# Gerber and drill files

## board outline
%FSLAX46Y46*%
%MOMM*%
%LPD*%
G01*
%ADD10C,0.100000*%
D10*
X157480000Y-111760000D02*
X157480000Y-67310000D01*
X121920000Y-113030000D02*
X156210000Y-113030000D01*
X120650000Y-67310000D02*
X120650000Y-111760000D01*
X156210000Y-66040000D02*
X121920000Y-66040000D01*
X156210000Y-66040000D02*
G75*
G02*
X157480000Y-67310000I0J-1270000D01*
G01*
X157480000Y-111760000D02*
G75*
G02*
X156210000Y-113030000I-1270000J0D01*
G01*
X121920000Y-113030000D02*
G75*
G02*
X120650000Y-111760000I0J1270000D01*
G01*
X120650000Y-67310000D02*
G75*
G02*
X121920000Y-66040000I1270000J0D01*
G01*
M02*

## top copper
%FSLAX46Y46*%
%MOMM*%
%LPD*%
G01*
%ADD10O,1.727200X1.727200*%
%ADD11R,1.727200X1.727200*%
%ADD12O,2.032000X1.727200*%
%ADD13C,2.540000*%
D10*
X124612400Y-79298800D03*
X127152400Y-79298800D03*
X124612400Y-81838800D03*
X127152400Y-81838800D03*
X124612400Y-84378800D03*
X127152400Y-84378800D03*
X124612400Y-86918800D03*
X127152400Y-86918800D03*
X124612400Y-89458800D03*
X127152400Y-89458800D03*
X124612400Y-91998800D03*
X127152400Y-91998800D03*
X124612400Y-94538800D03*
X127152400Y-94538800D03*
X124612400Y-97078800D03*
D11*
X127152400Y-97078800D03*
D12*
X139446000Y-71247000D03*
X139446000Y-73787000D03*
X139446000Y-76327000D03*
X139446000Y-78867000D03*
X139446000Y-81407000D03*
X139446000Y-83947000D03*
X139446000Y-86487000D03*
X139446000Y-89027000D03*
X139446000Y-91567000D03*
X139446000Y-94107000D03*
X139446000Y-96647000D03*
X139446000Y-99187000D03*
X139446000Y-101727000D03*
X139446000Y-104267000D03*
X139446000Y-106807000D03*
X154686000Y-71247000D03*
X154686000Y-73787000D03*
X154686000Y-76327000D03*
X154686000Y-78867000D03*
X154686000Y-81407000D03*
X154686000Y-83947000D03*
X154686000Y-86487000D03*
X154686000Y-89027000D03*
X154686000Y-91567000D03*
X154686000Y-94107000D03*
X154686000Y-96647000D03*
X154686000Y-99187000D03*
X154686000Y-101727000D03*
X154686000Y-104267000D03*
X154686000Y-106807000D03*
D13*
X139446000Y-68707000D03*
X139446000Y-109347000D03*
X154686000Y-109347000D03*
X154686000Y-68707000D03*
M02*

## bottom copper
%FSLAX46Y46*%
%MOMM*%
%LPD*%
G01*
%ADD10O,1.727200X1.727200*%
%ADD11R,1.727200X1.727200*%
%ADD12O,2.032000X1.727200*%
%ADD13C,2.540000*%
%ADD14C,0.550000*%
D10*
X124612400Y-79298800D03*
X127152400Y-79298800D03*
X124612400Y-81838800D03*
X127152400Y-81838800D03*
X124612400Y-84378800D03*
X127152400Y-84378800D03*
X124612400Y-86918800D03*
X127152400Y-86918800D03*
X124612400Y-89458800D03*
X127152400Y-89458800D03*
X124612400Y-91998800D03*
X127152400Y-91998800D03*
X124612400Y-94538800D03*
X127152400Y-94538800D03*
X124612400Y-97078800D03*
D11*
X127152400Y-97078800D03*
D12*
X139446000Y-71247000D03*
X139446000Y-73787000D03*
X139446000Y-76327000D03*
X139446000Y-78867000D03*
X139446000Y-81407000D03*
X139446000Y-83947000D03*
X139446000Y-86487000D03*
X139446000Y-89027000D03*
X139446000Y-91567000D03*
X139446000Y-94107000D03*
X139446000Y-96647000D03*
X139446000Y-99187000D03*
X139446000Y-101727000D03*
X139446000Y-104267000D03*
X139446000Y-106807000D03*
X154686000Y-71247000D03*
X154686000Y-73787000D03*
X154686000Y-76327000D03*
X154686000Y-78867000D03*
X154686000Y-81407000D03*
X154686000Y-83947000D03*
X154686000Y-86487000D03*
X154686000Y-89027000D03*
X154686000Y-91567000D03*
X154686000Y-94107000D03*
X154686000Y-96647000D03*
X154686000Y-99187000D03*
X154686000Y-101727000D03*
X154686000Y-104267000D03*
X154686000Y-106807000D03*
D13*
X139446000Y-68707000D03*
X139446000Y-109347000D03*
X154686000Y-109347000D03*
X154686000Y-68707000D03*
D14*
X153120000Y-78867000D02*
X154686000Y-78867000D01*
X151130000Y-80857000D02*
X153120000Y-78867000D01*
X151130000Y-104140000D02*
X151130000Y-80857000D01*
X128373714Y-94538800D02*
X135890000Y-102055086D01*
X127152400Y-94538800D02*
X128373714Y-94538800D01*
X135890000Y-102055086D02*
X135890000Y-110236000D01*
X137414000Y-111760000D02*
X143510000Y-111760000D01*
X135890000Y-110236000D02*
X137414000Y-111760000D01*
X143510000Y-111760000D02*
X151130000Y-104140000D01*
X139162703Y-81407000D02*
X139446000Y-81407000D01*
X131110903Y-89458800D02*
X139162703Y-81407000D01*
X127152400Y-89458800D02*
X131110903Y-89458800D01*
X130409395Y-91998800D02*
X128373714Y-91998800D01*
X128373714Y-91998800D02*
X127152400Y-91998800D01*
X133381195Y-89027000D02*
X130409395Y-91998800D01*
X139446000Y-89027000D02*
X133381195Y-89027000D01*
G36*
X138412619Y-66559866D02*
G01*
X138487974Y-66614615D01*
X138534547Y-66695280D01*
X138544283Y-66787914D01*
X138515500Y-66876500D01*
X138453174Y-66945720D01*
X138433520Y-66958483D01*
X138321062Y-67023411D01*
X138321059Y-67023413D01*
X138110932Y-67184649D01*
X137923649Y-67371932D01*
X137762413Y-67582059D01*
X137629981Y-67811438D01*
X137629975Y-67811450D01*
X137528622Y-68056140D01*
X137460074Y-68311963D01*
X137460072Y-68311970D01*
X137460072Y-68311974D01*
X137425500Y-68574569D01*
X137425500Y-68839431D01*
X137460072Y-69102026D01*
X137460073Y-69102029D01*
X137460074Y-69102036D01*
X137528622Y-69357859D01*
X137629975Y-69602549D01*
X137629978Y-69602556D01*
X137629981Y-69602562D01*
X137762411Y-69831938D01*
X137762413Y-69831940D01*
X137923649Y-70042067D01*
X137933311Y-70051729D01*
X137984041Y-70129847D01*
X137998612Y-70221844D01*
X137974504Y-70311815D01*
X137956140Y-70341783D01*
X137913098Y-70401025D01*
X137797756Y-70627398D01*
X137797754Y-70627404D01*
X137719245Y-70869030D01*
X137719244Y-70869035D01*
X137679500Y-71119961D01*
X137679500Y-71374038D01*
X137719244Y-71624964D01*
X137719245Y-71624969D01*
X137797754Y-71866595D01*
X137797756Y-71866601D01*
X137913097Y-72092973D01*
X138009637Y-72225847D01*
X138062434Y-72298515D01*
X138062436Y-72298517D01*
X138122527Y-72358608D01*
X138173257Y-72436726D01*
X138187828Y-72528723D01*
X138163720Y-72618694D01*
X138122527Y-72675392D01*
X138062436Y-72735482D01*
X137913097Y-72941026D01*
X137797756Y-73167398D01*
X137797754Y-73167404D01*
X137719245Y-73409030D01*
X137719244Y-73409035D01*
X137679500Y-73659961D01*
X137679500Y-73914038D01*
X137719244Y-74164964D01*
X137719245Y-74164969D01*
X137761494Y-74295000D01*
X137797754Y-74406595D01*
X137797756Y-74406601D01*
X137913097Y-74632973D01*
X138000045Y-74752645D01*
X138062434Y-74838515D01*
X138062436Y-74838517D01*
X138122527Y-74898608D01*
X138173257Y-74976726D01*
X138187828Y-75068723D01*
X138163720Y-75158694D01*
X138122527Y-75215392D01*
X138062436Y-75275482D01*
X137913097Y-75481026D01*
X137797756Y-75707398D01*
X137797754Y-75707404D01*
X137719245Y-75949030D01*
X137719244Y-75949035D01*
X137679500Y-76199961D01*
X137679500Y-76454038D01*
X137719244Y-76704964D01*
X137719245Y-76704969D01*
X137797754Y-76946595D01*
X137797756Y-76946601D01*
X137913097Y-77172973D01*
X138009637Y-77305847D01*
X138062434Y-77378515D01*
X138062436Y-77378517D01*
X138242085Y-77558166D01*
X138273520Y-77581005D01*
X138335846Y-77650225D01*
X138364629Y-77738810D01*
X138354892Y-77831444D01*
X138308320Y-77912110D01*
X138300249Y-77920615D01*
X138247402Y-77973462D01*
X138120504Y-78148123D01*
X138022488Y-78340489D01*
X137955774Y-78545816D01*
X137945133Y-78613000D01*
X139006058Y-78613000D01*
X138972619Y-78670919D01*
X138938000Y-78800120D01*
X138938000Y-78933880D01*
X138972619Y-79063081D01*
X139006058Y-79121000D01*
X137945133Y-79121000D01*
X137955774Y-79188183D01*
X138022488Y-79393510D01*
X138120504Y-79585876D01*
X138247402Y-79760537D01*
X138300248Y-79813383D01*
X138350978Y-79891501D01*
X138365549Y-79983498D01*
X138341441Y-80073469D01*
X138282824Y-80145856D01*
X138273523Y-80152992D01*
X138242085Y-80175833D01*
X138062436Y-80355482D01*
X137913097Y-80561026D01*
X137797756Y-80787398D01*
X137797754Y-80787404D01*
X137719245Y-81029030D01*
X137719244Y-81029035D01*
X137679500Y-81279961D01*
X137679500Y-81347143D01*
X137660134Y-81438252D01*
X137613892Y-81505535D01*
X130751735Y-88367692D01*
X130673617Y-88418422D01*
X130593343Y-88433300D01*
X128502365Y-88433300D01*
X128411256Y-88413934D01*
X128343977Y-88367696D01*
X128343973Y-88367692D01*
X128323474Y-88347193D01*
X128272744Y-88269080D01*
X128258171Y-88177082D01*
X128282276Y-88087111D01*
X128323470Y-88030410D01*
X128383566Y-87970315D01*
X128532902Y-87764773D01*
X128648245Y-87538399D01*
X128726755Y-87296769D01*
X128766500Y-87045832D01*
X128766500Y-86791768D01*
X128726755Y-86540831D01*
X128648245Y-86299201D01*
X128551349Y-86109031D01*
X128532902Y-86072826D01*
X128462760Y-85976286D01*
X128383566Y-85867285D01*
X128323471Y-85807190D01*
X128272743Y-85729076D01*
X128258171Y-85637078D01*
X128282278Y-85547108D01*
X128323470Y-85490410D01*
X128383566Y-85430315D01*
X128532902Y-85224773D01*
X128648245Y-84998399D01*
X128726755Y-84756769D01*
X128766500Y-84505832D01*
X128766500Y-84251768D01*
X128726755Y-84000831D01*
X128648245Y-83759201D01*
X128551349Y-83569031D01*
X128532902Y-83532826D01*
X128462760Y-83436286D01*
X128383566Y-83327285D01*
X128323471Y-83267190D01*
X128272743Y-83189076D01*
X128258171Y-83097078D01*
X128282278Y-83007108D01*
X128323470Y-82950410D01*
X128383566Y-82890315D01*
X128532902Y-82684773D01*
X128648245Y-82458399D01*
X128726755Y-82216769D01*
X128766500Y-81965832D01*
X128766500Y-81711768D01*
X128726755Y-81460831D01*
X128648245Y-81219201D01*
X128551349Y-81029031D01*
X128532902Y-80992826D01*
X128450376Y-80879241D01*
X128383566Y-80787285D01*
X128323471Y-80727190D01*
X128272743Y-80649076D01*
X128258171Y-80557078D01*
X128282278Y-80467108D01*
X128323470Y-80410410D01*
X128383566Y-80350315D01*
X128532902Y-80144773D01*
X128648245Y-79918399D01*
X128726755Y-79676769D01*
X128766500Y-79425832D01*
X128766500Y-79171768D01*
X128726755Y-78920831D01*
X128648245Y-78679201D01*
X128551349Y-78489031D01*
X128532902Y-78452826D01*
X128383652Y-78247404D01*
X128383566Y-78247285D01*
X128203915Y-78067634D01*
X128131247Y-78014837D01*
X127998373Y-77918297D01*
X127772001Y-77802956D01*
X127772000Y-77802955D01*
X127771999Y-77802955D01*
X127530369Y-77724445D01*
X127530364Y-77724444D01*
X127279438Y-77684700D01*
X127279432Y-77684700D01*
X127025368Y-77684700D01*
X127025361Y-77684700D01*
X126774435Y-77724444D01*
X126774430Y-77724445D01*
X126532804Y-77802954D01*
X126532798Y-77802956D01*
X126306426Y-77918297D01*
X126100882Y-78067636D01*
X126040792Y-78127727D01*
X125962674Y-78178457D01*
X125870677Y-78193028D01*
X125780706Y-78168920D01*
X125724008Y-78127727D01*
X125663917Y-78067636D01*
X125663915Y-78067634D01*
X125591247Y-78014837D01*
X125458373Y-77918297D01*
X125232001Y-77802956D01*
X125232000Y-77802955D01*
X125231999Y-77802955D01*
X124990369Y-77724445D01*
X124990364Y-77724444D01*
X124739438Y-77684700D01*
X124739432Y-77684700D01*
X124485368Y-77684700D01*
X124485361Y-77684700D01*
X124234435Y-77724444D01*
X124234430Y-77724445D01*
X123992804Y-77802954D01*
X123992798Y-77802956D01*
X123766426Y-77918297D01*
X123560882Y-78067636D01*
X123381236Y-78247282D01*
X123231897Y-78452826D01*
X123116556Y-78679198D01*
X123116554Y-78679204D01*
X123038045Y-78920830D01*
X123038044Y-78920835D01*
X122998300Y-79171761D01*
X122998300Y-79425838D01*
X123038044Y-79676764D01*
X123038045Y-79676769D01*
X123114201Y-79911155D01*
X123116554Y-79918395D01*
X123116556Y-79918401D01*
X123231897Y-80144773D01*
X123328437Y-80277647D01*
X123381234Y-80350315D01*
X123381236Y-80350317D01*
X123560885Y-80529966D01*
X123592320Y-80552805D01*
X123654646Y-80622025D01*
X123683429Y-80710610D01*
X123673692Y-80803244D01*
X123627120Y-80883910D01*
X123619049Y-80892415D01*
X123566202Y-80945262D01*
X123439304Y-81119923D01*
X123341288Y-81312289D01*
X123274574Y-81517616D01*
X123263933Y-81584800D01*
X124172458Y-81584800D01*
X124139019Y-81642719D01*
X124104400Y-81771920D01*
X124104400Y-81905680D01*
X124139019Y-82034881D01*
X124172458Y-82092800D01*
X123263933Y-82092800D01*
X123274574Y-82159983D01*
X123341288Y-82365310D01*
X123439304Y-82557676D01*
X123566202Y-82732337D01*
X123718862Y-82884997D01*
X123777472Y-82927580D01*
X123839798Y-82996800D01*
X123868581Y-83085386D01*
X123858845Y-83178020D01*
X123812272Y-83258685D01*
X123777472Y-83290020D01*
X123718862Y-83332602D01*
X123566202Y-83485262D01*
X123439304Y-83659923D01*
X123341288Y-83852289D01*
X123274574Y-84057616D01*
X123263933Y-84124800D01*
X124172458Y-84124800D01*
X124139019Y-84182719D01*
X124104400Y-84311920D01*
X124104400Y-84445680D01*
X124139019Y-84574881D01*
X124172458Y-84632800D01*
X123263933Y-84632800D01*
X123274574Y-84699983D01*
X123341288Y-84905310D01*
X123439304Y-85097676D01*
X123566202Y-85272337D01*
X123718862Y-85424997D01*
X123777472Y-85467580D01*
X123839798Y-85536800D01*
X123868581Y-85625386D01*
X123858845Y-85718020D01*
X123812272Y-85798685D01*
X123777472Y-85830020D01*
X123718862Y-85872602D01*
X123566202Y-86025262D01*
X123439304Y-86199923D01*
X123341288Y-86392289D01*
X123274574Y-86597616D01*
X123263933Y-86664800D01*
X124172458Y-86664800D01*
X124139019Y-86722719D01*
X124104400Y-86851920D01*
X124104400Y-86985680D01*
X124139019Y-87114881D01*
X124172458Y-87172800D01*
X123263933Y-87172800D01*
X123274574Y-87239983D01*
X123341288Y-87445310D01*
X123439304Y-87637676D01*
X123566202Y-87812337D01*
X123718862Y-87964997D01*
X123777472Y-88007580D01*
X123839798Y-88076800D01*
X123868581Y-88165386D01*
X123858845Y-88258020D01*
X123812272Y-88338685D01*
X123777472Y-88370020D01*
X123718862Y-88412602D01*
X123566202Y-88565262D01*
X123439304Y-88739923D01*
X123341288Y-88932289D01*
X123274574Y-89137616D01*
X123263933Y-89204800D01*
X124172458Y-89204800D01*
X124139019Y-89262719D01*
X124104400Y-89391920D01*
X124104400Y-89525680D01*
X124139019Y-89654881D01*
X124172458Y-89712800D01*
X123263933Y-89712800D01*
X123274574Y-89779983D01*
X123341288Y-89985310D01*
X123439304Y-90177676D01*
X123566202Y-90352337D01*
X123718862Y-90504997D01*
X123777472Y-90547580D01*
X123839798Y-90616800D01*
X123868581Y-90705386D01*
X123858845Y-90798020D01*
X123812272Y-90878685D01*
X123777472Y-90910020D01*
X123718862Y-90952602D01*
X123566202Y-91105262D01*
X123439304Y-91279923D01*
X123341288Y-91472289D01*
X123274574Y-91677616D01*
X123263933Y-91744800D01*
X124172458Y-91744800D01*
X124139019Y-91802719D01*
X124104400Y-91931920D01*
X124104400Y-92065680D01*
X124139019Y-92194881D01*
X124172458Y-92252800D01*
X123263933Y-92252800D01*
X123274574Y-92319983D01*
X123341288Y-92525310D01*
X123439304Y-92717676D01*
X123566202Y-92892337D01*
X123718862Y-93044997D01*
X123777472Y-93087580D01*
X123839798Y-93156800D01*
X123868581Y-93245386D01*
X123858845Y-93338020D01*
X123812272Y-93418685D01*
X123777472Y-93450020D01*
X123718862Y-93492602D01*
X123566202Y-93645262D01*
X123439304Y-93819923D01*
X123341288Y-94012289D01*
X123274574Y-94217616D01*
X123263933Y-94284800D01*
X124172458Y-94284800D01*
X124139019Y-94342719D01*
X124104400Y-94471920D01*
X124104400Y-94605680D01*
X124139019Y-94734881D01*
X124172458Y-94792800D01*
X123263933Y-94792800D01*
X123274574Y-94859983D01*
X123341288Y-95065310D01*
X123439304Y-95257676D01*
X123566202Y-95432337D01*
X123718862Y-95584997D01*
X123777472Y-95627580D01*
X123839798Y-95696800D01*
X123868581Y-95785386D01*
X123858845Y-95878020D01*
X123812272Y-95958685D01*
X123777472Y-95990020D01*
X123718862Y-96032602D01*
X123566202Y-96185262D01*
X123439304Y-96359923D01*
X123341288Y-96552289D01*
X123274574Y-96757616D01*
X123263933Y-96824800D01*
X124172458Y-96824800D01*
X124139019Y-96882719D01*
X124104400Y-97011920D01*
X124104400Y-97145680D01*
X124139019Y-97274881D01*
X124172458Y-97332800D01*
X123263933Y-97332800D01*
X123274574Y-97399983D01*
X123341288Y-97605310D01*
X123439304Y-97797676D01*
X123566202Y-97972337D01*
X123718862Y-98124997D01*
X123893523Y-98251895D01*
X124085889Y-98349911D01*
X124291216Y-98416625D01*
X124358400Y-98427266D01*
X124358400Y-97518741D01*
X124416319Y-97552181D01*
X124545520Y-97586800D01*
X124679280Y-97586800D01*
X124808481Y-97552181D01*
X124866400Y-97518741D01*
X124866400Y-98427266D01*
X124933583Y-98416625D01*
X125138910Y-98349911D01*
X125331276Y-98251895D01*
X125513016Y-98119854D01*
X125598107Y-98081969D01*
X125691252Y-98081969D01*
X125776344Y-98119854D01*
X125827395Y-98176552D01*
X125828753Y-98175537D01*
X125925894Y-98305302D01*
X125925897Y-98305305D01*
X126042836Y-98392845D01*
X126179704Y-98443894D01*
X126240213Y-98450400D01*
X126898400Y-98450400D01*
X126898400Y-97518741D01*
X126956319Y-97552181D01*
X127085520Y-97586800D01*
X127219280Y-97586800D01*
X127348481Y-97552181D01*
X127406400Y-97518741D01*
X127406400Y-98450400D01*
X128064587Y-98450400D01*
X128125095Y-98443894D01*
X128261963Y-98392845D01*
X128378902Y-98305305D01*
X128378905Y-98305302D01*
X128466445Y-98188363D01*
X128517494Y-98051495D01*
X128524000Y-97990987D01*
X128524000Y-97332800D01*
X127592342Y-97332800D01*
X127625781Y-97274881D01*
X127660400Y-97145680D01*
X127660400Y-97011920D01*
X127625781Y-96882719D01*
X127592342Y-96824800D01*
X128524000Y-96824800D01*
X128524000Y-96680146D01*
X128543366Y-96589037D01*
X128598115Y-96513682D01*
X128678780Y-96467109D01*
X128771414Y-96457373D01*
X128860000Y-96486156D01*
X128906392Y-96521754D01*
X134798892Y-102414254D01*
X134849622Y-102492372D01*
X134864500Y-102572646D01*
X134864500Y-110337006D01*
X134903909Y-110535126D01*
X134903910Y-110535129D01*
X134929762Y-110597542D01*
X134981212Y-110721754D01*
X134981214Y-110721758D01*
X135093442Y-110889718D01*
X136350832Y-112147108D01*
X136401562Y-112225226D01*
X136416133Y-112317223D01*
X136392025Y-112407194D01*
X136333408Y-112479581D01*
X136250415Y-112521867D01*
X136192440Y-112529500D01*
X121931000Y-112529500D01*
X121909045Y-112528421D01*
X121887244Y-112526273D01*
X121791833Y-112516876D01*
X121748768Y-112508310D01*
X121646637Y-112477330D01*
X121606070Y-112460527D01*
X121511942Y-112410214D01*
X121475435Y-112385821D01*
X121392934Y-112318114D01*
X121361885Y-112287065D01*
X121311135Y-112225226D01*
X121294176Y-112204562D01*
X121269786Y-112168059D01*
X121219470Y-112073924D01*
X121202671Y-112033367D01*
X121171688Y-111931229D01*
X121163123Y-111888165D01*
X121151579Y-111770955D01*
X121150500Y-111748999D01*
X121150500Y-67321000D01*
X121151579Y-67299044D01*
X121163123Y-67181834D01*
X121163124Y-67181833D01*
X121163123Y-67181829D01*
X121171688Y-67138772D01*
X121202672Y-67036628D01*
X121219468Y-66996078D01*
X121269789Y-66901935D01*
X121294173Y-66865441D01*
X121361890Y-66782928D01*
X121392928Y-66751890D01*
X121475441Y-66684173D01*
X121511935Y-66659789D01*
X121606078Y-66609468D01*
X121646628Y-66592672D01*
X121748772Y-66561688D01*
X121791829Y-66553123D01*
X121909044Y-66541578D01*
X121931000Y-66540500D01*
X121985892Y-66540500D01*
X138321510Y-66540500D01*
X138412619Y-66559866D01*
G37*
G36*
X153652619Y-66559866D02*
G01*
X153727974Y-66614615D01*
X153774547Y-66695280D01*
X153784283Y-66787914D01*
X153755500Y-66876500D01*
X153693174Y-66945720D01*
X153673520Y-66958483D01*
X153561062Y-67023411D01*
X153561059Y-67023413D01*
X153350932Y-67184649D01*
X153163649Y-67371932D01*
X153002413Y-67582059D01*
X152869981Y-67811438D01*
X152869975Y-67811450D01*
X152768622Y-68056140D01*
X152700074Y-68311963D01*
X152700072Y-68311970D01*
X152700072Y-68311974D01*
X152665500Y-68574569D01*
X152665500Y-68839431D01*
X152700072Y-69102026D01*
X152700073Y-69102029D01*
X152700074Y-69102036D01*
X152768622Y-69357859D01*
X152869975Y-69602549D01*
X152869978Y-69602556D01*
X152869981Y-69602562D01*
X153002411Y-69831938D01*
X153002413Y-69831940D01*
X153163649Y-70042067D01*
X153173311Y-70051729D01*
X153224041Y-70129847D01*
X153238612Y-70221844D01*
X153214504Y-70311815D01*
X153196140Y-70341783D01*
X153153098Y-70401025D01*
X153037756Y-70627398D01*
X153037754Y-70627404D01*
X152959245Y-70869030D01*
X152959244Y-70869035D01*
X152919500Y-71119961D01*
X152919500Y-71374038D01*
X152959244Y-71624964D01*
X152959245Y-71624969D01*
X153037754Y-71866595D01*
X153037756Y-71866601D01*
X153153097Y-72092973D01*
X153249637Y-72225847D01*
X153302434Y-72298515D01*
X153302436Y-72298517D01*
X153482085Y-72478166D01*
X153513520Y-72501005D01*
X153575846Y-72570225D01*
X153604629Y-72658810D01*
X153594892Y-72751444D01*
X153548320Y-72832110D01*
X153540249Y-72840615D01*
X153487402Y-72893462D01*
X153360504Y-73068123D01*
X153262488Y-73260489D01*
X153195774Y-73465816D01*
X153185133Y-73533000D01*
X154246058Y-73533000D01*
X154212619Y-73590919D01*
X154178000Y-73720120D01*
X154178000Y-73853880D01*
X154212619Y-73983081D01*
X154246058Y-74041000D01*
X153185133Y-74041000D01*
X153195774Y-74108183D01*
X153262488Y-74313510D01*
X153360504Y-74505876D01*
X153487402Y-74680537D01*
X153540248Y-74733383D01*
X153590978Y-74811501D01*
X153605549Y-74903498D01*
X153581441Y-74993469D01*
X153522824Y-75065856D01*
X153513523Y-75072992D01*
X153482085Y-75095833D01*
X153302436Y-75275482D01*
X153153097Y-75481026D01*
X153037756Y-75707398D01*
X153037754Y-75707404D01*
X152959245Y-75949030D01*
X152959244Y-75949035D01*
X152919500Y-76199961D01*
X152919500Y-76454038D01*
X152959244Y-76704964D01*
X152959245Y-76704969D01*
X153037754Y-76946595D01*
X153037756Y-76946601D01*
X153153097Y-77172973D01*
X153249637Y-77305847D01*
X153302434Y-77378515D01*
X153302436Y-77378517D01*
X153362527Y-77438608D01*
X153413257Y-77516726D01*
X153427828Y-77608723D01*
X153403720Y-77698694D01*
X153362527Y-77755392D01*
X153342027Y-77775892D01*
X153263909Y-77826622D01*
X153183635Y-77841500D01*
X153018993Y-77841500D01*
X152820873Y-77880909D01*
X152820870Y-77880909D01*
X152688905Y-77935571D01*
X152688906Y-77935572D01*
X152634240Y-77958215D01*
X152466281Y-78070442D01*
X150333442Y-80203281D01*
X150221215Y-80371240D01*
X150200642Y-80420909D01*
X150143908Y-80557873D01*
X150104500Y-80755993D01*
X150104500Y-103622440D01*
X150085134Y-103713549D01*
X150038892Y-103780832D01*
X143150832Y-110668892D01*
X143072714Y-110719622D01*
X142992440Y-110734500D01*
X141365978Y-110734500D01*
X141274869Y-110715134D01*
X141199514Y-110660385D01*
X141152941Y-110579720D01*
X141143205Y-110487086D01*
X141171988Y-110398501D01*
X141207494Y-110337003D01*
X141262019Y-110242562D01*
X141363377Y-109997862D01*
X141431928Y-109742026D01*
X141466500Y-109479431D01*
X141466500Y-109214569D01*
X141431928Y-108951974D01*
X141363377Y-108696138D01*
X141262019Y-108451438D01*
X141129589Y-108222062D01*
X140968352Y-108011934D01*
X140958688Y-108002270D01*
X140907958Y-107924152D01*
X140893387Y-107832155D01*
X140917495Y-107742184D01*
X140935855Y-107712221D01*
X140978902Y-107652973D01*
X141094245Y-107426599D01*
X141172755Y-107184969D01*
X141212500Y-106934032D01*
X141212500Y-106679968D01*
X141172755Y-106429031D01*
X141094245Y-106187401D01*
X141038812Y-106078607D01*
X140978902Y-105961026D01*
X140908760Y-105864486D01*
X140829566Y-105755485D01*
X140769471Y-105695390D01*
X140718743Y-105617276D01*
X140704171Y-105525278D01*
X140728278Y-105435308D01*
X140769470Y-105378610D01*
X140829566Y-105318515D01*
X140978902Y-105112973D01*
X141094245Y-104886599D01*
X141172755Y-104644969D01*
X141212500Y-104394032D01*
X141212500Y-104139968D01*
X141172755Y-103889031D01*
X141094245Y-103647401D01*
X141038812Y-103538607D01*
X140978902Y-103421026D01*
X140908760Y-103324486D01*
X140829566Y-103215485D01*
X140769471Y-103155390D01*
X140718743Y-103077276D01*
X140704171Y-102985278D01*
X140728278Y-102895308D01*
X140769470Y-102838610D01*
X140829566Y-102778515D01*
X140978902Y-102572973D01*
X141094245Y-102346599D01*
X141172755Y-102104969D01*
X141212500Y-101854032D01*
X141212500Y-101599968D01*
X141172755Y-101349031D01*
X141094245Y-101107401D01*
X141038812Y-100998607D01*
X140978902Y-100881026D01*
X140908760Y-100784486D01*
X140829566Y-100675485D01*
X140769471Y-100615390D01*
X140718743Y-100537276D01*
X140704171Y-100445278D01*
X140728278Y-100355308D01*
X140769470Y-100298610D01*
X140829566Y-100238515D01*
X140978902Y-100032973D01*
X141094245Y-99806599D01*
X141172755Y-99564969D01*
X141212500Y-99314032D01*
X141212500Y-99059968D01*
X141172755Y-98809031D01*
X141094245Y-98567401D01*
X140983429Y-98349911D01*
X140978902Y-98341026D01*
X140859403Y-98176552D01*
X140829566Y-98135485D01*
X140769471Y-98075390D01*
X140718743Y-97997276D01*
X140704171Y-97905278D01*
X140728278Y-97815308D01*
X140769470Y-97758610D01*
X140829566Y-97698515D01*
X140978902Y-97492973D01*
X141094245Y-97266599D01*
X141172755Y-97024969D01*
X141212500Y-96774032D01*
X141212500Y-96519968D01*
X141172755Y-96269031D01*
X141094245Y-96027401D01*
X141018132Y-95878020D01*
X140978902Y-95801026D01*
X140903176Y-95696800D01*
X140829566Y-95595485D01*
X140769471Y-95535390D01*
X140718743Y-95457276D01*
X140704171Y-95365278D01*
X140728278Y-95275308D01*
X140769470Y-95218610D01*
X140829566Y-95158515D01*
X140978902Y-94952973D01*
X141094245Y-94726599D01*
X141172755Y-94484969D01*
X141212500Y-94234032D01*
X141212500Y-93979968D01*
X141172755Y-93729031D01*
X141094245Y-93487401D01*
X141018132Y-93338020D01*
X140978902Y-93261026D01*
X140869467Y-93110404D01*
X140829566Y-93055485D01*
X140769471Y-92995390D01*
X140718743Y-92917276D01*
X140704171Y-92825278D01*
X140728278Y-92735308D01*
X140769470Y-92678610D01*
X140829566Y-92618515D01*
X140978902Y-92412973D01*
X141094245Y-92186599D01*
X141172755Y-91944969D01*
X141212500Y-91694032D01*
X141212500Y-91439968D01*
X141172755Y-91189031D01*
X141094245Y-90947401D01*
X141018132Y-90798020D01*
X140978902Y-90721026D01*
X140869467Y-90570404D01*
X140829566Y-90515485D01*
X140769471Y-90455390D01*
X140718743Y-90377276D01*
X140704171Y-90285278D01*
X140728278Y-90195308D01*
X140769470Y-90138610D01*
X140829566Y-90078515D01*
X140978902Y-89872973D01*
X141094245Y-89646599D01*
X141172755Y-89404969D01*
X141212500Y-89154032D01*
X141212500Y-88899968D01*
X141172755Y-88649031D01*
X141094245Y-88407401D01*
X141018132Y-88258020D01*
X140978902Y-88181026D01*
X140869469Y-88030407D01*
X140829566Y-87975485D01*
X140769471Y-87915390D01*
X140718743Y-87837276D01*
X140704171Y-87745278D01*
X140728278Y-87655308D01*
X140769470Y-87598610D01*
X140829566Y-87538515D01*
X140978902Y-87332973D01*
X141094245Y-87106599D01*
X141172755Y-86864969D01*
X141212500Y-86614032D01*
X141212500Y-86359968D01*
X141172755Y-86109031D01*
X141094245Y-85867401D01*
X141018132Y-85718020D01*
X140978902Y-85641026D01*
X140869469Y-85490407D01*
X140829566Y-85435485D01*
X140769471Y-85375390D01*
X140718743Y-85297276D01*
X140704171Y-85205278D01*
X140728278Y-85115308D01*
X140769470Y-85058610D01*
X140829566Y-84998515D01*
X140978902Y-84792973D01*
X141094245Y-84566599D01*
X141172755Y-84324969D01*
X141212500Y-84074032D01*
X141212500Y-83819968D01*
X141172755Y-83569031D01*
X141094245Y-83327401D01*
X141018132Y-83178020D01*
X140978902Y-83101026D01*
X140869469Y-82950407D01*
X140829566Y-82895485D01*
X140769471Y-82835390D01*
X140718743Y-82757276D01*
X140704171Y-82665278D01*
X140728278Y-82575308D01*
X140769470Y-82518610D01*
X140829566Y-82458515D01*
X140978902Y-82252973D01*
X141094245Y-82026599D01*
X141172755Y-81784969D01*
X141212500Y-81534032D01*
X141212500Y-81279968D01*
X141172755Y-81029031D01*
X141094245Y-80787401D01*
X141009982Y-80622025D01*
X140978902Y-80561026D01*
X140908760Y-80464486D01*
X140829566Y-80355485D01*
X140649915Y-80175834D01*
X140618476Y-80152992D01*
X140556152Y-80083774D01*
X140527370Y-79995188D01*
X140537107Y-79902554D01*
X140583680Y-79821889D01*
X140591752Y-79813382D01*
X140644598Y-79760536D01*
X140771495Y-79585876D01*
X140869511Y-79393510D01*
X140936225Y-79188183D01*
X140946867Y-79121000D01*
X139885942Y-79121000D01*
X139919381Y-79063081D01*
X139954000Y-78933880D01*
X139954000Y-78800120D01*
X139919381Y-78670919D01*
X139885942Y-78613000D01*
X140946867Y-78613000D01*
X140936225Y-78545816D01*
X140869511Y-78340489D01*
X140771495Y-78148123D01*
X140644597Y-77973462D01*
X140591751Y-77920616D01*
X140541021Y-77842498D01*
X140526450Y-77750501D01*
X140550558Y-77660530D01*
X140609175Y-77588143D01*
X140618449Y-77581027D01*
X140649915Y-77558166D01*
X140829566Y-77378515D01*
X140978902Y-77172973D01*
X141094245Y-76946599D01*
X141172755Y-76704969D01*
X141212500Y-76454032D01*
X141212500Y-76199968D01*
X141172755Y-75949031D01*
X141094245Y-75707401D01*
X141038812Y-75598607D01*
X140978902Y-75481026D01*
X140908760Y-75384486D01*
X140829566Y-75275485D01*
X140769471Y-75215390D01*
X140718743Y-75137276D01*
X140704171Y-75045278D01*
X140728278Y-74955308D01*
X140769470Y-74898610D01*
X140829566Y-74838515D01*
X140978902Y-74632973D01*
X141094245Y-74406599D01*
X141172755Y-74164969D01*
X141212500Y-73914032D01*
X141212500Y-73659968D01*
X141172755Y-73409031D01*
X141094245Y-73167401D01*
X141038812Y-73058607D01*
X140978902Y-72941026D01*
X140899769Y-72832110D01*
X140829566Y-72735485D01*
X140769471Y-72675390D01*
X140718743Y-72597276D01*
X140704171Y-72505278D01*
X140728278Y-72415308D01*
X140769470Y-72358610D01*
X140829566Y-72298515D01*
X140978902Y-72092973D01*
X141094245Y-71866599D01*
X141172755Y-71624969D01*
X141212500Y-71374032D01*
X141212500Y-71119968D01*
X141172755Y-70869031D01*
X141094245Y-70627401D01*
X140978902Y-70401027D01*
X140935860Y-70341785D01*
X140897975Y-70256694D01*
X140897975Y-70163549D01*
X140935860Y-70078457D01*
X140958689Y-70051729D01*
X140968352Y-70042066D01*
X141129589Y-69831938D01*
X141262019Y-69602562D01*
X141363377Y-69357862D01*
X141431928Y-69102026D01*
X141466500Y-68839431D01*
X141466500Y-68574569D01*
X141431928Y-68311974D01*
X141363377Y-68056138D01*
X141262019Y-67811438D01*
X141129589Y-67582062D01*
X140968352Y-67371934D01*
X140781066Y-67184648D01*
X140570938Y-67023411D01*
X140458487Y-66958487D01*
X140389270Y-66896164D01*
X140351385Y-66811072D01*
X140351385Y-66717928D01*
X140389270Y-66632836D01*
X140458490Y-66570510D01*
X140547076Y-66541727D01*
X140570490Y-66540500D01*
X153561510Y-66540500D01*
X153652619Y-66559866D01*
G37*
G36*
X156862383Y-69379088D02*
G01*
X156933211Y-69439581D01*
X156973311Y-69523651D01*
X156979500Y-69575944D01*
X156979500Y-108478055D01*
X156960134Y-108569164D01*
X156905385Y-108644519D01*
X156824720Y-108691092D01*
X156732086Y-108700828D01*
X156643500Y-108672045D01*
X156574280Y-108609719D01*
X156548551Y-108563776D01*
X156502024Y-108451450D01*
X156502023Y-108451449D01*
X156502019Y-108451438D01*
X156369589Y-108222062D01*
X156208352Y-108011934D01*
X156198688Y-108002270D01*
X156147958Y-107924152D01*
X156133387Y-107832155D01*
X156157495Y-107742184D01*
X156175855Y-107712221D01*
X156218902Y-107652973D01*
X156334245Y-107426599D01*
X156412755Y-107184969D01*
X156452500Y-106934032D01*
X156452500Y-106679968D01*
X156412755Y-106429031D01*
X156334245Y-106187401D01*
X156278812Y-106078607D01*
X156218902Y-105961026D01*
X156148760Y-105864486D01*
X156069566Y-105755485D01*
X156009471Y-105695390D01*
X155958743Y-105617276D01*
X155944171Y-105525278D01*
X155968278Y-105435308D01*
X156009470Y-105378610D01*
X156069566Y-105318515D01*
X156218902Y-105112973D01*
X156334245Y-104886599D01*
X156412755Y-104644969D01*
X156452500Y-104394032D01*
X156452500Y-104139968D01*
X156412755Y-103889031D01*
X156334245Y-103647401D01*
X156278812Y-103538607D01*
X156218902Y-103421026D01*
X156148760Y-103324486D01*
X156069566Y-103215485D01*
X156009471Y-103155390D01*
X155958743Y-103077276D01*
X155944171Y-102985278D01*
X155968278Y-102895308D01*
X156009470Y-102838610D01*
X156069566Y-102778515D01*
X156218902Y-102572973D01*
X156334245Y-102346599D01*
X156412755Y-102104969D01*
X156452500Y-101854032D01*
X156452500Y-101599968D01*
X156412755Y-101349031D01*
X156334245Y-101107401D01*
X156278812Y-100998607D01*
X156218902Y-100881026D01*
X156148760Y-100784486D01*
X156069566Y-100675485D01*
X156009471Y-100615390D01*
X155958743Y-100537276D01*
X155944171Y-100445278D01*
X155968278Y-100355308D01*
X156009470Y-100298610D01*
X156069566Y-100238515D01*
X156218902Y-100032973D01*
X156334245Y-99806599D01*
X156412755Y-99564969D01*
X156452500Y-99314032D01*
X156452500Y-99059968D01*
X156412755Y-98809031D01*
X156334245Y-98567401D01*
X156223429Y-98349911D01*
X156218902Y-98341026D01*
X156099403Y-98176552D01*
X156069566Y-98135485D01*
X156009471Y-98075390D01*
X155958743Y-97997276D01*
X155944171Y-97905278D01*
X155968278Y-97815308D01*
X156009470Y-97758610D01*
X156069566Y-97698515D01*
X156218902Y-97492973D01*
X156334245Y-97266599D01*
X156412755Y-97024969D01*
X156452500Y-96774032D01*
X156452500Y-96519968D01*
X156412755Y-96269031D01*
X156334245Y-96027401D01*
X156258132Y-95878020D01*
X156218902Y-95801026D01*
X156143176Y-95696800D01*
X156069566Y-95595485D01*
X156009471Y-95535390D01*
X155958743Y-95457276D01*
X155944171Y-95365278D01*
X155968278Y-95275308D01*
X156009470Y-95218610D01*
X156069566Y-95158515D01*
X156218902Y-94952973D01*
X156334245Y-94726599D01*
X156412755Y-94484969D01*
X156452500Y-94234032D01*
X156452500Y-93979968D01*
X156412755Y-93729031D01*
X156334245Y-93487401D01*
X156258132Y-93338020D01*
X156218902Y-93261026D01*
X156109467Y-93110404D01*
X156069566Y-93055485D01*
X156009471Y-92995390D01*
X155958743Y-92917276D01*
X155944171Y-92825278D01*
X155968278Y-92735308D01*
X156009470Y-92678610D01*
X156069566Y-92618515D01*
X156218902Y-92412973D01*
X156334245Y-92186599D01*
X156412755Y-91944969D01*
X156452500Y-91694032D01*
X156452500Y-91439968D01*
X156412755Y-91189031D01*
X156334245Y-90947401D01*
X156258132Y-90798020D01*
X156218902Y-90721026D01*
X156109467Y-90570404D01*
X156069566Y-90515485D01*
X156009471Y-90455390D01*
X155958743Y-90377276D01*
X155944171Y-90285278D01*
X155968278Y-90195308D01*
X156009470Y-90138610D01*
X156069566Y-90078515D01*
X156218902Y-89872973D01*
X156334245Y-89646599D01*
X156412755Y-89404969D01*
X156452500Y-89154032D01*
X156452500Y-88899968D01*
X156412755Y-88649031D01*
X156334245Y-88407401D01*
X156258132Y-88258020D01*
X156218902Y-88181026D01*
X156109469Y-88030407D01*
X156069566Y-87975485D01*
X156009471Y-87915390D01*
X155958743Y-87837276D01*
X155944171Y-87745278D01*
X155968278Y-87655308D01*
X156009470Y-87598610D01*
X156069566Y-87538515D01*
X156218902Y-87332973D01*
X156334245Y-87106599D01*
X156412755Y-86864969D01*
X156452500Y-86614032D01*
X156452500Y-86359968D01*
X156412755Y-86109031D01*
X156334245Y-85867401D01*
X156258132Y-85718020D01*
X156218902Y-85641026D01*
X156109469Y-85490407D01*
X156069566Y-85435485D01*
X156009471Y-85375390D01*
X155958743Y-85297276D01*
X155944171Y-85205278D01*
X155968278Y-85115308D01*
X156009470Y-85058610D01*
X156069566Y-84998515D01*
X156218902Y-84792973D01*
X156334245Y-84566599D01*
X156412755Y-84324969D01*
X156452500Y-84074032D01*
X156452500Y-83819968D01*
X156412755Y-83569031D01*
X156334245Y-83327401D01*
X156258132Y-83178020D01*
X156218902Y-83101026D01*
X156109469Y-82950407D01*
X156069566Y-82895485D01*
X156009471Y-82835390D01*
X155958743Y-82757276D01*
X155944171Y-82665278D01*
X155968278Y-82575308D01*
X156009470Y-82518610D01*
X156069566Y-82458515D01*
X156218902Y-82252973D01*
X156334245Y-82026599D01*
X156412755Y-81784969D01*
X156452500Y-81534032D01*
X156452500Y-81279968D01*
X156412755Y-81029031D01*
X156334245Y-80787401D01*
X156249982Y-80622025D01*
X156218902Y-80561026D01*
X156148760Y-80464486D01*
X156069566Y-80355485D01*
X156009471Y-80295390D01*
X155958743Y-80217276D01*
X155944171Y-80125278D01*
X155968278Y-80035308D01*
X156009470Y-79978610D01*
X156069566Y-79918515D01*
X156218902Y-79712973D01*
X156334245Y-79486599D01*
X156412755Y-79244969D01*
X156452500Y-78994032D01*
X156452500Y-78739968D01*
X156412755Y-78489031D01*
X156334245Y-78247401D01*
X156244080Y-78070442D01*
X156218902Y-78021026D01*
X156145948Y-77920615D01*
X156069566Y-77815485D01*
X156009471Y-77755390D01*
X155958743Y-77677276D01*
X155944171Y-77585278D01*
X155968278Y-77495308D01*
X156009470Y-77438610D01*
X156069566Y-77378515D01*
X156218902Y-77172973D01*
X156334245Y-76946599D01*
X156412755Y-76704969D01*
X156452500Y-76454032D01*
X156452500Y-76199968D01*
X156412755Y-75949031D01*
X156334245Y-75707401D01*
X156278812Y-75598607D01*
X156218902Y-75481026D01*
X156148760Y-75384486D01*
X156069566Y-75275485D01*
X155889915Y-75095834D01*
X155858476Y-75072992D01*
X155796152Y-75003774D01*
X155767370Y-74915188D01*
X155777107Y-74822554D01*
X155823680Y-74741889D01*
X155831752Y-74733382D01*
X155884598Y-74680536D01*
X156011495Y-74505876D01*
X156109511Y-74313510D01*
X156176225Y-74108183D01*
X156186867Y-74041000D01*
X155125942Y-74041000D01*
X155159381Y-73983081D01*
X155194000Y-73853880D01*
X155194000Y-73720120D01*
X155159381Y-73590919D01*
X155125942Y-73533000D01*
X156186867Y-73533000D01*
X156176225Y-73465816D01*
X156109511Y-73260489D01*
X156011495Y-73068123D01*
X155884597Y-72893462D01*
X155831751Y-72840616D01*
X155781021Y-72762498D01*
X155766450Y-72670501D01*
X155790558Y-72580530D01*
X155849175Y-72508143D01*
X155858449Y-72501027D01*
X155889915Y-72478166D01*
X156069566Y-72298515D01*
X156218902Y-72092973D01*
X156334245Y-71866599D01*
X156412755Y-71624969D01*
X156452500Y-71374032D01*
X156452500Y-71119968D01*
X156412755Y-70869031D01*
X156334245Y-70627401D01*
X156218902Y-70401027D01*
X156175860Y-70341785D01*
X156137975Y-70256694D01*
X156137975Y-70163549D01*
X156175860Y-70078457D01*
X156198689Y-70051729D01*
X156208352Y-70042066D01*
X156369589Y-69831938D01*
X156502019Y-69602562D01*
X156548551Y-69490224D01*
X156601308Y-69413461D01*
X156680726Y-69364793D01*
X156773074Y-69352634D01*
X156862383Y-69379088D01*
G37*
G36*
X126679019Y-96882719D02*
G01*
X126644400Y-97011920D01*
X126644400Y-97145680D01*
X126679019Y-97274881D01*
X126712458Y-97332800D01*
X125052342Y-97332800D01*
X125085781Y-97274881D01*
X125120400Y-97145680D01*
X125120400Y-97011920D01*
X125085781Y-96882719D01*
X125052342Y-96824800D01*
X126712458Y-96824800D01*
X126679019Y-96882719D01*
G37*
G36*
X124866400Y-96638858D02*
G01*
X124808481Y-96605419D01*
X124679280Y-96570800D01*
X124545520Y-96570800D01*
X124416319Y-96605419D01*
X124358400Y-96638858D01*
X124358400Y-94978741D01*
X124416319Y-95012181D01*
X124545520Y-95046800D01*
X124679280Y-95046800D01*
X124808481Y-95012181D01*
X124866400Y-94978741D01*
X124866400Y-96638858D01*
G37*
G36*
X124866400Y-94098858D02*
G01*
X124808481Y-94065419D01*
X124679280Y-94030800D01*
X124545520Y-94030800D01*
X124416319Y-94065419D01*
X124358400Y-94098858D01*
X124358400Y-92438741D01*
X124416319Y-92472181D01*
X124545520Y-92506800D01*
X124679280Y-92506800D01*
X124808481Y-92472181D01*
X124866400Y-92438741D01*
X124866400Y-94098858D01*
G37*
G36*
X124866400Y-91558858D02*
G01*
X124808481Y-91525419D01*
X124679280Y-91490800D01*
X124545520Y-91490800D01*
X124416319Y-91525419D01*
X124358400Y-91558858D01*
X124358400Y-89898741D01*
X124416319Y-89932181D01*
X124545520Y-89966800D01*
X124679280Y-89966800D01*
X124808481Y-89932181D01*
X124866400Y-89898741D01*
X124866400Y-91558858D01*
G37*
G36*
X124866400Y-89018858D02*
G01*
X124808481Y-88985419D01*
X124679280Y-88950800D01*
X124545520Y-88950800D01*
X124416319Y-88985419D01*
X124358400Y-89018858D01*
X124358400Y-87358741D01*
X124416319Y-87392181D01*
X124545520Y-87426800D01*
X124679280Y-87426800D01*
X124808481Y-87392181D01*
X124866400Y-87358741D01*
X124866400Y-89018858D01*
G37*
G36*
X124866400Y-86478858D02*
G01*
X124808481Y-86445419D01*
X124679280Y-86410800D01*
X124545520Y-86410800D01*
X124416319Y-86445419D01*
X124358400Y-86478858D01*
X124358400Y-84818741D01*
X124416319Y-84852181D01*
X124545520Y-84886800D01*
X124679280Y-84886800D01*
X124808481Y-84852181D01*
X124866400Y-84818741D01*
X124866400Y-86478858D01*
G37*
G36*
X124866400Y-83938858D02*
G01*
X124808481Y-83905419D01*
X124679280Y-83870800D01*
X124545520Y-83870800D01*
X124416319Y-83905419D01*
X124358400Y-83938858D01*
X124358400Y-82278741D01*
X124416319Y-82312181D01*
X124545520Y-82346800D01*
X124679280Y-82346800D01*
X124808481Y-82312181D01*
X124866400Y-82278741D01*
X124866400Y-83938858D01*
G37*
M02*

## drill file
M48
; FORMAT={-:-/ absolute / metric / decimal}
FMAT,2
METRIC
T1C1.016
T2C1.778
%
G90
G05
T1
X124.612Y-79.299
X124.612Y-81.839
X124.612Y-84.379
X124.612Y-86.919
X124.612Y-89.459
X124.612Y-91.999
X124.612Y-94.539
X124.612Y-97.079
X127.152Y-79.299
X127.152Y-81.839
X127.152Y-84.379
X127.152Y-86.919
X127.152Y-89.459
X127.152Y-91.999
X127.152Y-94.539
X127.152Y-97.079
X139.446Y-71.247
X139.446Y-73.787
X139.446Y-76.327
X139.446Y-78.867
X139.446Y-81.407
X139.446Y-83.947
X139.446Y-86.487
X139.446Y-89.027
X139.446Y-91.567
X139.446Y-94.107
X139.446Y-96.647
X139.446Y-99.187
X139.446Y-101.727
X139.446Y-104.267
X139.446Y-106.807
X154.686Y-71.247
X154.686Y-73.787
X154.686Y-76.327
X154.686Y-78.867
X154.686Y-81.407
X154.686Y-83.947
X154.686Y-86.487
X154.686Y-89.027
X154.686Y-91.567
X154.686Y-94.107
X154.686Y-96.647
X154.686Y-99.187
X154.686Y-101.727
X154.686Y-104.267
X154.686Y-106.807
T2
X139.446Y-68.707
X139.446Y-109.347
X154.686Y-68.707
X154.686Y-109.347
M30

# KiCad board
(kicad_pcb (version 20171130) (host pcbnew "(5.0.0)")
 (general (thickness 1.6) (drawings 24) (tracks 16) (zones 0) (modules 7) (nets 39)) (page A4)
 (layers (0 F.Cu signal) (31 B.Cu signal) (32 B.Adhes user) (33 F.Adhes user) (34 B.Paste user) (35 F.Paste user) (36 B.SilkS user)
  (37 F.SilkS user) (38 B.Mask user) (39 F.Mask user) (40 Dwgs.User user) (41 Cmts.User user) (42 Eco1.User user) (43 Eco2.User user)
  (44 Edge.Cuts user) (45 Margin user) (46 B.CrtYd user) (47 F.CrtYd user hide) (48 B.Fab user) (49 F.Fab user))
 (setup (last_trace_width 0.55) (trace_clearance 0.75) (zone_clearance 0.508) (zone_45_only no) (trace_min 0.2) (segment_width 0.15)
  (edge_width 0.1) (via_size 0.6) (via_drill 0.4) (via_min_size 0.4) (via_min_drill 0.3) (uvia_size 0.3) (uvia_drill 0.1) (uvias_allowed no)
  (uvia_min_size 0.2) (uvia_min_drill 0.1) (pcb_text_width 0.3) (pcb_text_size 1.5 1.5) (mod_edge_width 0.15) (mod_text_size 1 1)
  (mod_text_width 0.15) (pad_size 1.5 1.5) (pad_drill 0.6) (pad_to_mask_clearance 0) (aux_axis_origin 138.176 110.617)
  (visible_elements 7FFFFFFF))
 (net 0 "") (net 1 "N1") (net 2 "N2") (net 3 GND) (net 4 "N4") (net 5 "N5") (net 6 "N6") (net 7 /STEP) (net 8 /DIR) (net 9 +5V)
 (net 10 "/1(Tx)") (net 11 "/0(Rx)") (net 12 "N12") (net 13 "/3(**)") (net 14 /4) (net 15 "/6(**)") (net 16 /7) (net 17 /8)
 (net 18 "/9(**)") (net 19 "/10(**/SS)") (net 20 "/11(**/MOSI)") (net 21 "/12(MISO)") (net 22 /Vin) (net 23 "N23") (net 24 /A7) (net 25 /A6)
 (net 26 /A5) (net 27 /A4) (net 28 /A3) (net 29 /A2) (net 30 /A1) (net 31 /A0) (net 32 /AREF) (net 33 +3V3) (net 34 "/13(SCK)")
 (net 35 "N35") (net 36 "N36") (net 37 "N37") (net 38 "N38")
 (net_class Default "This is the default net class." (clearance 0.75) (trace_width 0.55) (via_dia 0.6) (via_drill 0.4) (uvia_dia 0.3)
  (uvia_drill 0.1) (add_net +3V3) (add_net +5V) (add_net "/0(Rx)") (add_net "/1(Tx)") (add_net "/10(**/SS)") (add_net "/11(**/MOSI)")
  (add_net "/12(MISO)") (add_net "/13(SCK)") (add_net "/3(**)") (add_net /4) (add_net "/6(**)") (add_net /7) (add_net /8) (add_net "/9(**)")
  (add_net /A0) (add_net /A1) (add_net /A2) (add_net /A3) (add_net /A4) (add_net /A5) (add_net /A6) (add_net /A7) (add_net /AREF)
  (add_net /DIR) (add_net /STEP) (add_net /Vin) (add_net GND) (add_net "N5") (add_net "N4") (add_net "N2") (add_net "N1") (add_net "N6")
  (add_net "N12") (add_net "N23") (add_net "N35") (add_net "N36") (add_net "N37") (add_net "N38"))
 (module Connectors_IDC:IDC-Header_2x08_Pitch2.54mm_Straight (layer F.Cu) (at 127.1524 97.0788 180)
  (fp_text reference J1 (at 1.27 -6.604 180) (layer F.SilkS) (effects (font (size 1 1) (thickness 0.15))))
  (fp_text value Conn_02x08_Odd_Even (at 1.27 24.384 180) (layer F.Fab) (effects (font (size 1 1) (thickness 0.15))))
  (pad 16 thru_hole oval (at 2.54 17.78 180) (size 1.7272 1.7272) (drill 1.016) (layers *.Cu *.Mask) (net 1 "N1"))
  (pad 15 thru_hole oval (at 0 17.78 180) (size 1.7272 1.7272) (drill 1.016) (layers *.Cu *.Mask) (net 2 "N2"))
  (pad 14 thru_hole oval (at 2.54 15.24 180) (size 1.7272 1.7272) (drill 1.016) (layers *.Cu *.Mask) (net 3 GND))
  (pad 13 thru_hole oval (at 0 15.24 180) (size 1.7272 1.7272) (drill 1.016) (layers *.Cu *.Mask) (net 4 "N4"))
  (pad 12 thru_hole oval (at 2.54 12.7 180) (size 1.7272 1.7272) (drill 1.016) (layers *.Cu *.Mask) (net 3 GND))
  (pad 11 thru_hole oval (at 0 12.7 180) (size 1.7272 1.7272) (drill 1.016) (layers *.Cu *.Mask) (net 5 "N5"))
  (pad 10 thru_hole oval (at 2.54 10.16 180) (size 1.7272 1.7272) (drill 1.016) (layers *.Cu *.Mask) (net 3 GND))
  (pad 9 thru_hole oval (at 0 10.16 180) (size 1.7272 1.7272) (drill 1.016) (layers *.Cu *.Mask) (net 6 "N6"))
  (pad 8 thru_hole oval (at 2.54 7.62 180) (size 1.7272 1.7272) (drill 1.016) (layers *.Cu *.Mask) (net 3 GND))
  (pad 7 thru_hole oval (at 0 7.62 180) (size 1.7272 1.7272) (drill 1.016) (layers *.Cu *.Mask) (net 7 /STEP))
  (pad 6 thru_hole oval (at 2.54 5.08 180) (size 1.7272 1.7272) (drill 1.016) (layers *.Cu *.Mask) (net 3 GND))
  (pad 5 thru_hole oval (at 0 5.08 180) (size 1.7272 1.7272) (drill 1.016) (layers *.Cu *.Mask) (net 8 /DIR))
  (pad 4 thru_hole oval (at 2.54 2.54 180) (size 1.7272 1.7272) (drill 1.016) (layers *.Cu *.Mask) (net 3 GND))
  (pad 3 thru_hole oval (at 0 2.54 180) (size 1.7272 1.7272) (drill 1.016) (layers *.Cu *.Mask) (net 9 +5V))
  (pad 2 thru_hole oval (at 2.54 0 180) (size 1.7272 1.7272) (drill 1.016) (layers *.Cu *.Mask) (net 3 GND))
  (pad 1 thru_hole rect (at 0 0 180) (size 1.7272 1.7272) (drill 1.016) (layers *.Cu *.Mask) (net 3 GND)))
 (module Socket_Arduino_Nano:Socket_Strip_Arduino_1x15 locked (layer F.Cu) (at 139.446 71.247 270)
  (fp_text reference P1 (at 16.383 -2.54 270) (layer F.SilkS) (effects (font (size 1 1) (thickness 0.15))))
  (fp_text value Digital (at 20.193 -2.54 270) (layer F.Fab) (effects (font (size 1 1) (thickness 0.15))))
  (pad 1 thru_hole oval (at 0 0 270) (size 1.7272 2.032) (drill 1.016) (layers *.Cu *.Mask F.SilkS) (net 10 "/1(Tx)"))
  (pad 2 thru_hole oval (at 2.54 0 270) (size 1.7272 2.032) (drill 1.016) (layers *.Cu *.Mask F.SilkS) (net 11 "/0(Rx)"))
  (pad 3 thru_hole oval (at 5.08 0 270) (size 1.7272 2.032) (drill 1.016) (layers *.Cu *.Mask F.SilkS) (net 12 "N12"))
  (pad 4 thru_hole oval (at 7.62 0 270) (size 1.7272 2.032) (drill 1.016) (layers *.Cu *.Mask F.SilkS) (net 3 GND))
  (pad 5 thru_hole oval (at 10.16 0 270) (size 1.7272 2.032) (drill 1.016) (layers *.Cu *.Mask F.SilkS) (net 7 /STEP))
  (pad 6 thru_hole oval (at 12.7 0 270) (size 1.7272 2.032) (drill 1.016) (layers *.Cu *.Mask F.SilkS) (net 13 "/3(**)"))
  (pad 7 thru_hole oval (at 15.24 0 270) (size 1.7272 2.032) (drill 1.016) (layers *.Cu *.Mask F.SilkS) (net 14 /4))
  (pad 8 thru_hole oval (at 17.78 0 270) (size 1.7272 2.032) (drill 1.016) (layers *.Cu *.Mask F.SilkS) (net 8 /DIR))
  (pad 9 thru_hole oval (at 20.32 0 270) (size 1.7272 2.032) (drill 1.016) (layers *.Cu *.Mask F.SilkS) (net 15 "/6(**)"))
  (pad 10 thru_hole oval (at 22.86 0 270) (size 1.7272 2.032) (drill 1.016) (layers *.Cu *.Mask F.SilkS) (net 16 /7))
  (pad 11 thru_hole oval (at 25.4 0 270) (size 1.7272 2.032) (drill 1.016) (layers *.Cu *.Mask F.SilkS) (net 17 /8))
  (pad 12 thru_hole oval (at 27.94 0 270) (size 1.7272 2.032) (drill 1.016) (layers *.Cu *.Mask F.SilkS) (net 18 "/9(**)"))
  (pad 13 thru_hole oval (at 30.48 0 270) (size 1.7272 2.032) (drill 1.016) (layers *.Cu *.Mask F.SilkS) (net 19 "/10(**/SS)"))
  (pad 14 thru_hole oval (at 33.02 0 270) (size 1.7272 2.032) (drill 1.016) (layers *.Cu *.Mask F.SilkS) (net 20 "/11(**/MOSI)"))
  (pad 15 thru_hole oval (at 35.56 0 270) (size 1.7272 2.032) (drill 1.016) (layers *.Cu *.Mask F.SilkS) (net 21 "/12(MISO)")))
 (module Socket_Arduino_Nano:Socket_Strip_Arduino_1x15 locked (layer F.Cu) (at 154.686 71.247 270)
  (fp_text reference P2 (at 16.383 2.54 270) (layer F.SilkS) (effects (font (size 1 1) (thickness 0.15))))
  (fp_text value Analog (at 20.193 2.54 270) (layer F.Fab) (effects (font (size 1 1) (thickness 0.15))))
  (pad 1 thru_hole oval (at 0 0 270) (size 1.7272 2.032) (drill 1.016) (layers *.Cu *.Mask F.SilkS) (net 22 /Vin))
  (pad 2 thru_hole oval (at 2.54 0 270) (size 1.7272 2.032) (drill 1.016) (layers *.Cu *.Mask F.SilkS) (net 3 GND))
  (pad 3 thru_hole oval (at 5.08 0 270) (size 1.7272 2.032) (drill 1.016) (layers *.Cu *.Mask F.SilkS) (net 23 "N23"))
  (pad 4 thru_hole oval (at 7.62 0 270) (size 1.7272 2.032) (drill 1.016) (layers *.Cu *.Mask F.SilkS) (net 9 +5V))
  (pad 5 thru_hole oval (at 10.16 0 270) (size 1.7272 2.032) (drill 1.016) (layers *.Cu *.Mask F.SilkS) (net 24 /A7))
  (pad 6 thru_hole oval (at 12.7 0 270) (size 1.7272 2.032) (drill 1.016) (layers *.Cu *.Mask F.SilkS) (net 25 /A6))
  (pad 7 thru_hole oval (at 15.24 0 270) (size 1.7272 2.032) (drill 1.016) (layers *.Cu *.Mask F.SilkS) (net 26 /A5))
  (pad 8 thru_hole oval (at 17.78 0 270) (size 1.7272 2.032) (drill 1.016) (layers *.Cu *.Mask F.SilkS) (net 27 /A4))
  (pad 9 thru_hole oval (at 20.32 0 270) (size 1.7272 2.032) (drill 1.016) (layers *.Cu *.Mask F.SilkS) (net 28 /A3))
  (pad 10 thru_hole oval (at 22.86 0 270) (size 1.7272 2.032) (drill 1.016) (layers *.Cu *.Mask F.SilkS) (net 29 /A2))
  (pad 11 thru_hole oval (at 25.4 0 270) (size 1.7272 2.032) (drill 1.016) (layers *.Cu *.Mask F.SilkS) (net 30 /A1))
  (pad 12 thru_hole oval (at 27.94 0 270) (size 1.7272 2.032) (drill 1.016) (layers *.Cu *.Mask F.SilkS) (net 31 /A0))
  (pad 13 thru_hole oval (at 30.48 0 270) (size 1.7272 2.032) (drill 1.016) (layers *.Cu *.Mask F.SilkS) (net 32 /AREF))
  (pad 14 thru_hole oval (at 33.02 0 270) (size 1.7272 2.032) (drill 1.016) (layers *.Cu *.Mask F.SilkS) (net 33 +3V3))
  (pad 15 thru_hole oval (at 35.56 0 270) (size 1.7272 2.032) (drill 1.016) (layers *.Cu *.Mask F.SilkS) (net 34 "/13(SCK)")))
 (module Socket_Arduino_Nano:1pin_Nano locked (layer F.Cu) (at 139.446 68.707)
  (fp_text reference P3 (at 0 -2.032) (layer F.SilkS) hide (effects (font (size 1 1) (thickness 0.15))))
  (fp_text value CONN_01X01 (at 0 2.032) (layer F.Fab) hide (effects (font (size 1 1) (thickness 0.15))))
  (pad 1 thru_hole circle (at 0 0) (size 2.54 2.54) (drill 1.778) (layers *.Cu *.Mask F.SilkS) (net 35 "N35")))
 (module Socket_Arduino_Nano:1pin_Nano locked (layer F.Cu) (at 139.446 109.347)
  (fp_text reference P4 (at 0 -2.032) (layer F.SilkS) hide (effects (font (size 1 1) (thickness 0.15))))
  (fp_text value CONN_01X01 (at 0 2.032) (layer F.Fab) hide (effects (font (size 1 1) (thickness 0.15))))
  (pad 1 thru_hole circle (at 0 0) (size 2.54 2.54) (drill 1.778) (layers *.Cu *.Mask F.SilkS) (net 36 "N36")))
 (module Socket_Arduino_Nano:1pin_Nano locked (layer F.Cu) (at 154.686 109.347)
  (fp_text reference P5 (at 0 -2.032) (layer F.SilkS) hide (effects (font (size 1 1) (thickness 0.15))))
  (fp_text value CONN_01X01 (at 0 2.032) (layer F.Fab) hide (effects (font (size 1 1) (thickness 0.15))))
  (pad 1 thru_hole circle (at 0 0) (size 2.54 2.54) (drill 1.778) (layers *.Cu *.Mask F.SilkS) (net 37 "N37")))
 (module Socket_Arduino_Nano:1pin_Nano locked (layer F.Cu) (at 154.686 68.707)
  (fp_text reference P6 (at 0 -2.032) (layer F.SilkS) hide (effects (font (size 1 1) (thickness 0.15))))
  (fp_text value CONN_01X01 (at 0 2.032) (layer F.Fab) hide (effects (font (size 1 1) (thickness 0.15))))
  (pad 1 thru_hole circle (at 0 0) (size 2.54 2.54) (drill 1.778) (layers *.Cu *.Mask F.SilkS) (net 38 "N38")))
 (gr_line (start 157.48 111.76) (end 157.48 67.31) (layer Edge.Cuts) (width 0.1))
 (gr_line (start 121.92 113.03) (end 156.21 113.03) (layer Edge.Cuts) (width 0.1))
 (gr_line (start 120.65 67.31) (end 120.65 111.76) (layer Edge.Cuts) (width 0.1))
 (gr_line (start 156.21 66.04) (end 121.92 66.04) (layer Edge.Cuts) (width 0.1))
 (gr_arc (start 156.21 67.31) (end 157.48 67.31) (angle -90) (layer Edge.Cuts) (width 0.1))
 (gr_arc (start 156.21 111.76) (end 156.21 113.03) (angle -90) (layer Edge.Cuts) (width 0.1))
 (gr_arc (start 121.92 111.76) (end 120.65 111.76) (angle -90) (layer Edge.Cuts) (width 0.1))
 (gr_arc (start 121.92 67.31) (end 121.92 66.04) (angle -90) (layer Edge.Cuts) (width 0.1))
 (segment (start 153.12 78.867) (end 154.686 78.867) (width 0.55) (layer B.Cu) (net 9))
 (segment (start 151.13 80.857) (end 153.12 78.867) (width 0.55) (layer B.Cu) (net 9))
 (segment (start 151.13 104.14) (end 151.13 80.857) (width 0.55) (layer B.Cu) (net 9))
 (segment (start 128.373714 94.5388) (end 135.89 102.055086) (width 0.55) (layer B.Cu) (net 9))
 (segment (start 127.1524 94.5388) (end 128.373714 94.5388) (width 0.55) (layer B.Cu) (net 9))
 (segment (start 135.89 102.055086) (end 135.89 110.236) (width 0.55) (layer B.Cu) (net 9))
 (segment (start 137.414 111.76) (end 143.51 111.76) (width 0.55) (layer B.Cu) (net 9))
 (segment (start 135.89 110.236) (end 137.414 111.76) (width 0.55) (layer B.Cu) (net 9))
 (segment (start 143.51 111.76) (end 151.13 104.14) (width 0.55) (layer B.Cu) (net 9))
 (segment (start 139.162703 81.407) (end 139.446 81.407) (width 0.55) (layer B.Cu) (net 7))
 (segment (start 131.110903 89.4588) (end 139.162703 81.407) (width 0.55) (layer B.Cu) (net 7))
 (segment (start 127.1524 89.4588) (end 131.110903 89.4588) (width 0.55) (layer B.Cu) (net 7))
 (segment (start 130.409395 91.9988) (end 128.373714 91.9988) (width 0.55) (layer B.Cu) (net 8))
 (segment (start 128.373714 91.9988) (end 127.1524 91.9988) (width 0.55) (layer B.Cu) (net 8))
 (segment (start 133.381195 89.027) (end 130.409395 91.9988) (width 0.55) (layer B.Cu) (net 8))
 (segment (start 139.446 89.027) (end 133.381195 89.027) (width 0.55) (layer B.Cu) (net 8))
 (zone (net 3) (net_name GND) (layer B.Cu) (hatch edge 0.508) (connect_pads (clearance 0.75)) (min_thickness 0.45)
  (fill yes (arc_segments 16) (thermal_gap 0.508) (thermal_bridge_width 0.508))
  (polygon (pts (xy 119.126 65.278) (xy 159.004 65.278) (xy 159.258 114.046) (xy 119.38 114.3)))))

